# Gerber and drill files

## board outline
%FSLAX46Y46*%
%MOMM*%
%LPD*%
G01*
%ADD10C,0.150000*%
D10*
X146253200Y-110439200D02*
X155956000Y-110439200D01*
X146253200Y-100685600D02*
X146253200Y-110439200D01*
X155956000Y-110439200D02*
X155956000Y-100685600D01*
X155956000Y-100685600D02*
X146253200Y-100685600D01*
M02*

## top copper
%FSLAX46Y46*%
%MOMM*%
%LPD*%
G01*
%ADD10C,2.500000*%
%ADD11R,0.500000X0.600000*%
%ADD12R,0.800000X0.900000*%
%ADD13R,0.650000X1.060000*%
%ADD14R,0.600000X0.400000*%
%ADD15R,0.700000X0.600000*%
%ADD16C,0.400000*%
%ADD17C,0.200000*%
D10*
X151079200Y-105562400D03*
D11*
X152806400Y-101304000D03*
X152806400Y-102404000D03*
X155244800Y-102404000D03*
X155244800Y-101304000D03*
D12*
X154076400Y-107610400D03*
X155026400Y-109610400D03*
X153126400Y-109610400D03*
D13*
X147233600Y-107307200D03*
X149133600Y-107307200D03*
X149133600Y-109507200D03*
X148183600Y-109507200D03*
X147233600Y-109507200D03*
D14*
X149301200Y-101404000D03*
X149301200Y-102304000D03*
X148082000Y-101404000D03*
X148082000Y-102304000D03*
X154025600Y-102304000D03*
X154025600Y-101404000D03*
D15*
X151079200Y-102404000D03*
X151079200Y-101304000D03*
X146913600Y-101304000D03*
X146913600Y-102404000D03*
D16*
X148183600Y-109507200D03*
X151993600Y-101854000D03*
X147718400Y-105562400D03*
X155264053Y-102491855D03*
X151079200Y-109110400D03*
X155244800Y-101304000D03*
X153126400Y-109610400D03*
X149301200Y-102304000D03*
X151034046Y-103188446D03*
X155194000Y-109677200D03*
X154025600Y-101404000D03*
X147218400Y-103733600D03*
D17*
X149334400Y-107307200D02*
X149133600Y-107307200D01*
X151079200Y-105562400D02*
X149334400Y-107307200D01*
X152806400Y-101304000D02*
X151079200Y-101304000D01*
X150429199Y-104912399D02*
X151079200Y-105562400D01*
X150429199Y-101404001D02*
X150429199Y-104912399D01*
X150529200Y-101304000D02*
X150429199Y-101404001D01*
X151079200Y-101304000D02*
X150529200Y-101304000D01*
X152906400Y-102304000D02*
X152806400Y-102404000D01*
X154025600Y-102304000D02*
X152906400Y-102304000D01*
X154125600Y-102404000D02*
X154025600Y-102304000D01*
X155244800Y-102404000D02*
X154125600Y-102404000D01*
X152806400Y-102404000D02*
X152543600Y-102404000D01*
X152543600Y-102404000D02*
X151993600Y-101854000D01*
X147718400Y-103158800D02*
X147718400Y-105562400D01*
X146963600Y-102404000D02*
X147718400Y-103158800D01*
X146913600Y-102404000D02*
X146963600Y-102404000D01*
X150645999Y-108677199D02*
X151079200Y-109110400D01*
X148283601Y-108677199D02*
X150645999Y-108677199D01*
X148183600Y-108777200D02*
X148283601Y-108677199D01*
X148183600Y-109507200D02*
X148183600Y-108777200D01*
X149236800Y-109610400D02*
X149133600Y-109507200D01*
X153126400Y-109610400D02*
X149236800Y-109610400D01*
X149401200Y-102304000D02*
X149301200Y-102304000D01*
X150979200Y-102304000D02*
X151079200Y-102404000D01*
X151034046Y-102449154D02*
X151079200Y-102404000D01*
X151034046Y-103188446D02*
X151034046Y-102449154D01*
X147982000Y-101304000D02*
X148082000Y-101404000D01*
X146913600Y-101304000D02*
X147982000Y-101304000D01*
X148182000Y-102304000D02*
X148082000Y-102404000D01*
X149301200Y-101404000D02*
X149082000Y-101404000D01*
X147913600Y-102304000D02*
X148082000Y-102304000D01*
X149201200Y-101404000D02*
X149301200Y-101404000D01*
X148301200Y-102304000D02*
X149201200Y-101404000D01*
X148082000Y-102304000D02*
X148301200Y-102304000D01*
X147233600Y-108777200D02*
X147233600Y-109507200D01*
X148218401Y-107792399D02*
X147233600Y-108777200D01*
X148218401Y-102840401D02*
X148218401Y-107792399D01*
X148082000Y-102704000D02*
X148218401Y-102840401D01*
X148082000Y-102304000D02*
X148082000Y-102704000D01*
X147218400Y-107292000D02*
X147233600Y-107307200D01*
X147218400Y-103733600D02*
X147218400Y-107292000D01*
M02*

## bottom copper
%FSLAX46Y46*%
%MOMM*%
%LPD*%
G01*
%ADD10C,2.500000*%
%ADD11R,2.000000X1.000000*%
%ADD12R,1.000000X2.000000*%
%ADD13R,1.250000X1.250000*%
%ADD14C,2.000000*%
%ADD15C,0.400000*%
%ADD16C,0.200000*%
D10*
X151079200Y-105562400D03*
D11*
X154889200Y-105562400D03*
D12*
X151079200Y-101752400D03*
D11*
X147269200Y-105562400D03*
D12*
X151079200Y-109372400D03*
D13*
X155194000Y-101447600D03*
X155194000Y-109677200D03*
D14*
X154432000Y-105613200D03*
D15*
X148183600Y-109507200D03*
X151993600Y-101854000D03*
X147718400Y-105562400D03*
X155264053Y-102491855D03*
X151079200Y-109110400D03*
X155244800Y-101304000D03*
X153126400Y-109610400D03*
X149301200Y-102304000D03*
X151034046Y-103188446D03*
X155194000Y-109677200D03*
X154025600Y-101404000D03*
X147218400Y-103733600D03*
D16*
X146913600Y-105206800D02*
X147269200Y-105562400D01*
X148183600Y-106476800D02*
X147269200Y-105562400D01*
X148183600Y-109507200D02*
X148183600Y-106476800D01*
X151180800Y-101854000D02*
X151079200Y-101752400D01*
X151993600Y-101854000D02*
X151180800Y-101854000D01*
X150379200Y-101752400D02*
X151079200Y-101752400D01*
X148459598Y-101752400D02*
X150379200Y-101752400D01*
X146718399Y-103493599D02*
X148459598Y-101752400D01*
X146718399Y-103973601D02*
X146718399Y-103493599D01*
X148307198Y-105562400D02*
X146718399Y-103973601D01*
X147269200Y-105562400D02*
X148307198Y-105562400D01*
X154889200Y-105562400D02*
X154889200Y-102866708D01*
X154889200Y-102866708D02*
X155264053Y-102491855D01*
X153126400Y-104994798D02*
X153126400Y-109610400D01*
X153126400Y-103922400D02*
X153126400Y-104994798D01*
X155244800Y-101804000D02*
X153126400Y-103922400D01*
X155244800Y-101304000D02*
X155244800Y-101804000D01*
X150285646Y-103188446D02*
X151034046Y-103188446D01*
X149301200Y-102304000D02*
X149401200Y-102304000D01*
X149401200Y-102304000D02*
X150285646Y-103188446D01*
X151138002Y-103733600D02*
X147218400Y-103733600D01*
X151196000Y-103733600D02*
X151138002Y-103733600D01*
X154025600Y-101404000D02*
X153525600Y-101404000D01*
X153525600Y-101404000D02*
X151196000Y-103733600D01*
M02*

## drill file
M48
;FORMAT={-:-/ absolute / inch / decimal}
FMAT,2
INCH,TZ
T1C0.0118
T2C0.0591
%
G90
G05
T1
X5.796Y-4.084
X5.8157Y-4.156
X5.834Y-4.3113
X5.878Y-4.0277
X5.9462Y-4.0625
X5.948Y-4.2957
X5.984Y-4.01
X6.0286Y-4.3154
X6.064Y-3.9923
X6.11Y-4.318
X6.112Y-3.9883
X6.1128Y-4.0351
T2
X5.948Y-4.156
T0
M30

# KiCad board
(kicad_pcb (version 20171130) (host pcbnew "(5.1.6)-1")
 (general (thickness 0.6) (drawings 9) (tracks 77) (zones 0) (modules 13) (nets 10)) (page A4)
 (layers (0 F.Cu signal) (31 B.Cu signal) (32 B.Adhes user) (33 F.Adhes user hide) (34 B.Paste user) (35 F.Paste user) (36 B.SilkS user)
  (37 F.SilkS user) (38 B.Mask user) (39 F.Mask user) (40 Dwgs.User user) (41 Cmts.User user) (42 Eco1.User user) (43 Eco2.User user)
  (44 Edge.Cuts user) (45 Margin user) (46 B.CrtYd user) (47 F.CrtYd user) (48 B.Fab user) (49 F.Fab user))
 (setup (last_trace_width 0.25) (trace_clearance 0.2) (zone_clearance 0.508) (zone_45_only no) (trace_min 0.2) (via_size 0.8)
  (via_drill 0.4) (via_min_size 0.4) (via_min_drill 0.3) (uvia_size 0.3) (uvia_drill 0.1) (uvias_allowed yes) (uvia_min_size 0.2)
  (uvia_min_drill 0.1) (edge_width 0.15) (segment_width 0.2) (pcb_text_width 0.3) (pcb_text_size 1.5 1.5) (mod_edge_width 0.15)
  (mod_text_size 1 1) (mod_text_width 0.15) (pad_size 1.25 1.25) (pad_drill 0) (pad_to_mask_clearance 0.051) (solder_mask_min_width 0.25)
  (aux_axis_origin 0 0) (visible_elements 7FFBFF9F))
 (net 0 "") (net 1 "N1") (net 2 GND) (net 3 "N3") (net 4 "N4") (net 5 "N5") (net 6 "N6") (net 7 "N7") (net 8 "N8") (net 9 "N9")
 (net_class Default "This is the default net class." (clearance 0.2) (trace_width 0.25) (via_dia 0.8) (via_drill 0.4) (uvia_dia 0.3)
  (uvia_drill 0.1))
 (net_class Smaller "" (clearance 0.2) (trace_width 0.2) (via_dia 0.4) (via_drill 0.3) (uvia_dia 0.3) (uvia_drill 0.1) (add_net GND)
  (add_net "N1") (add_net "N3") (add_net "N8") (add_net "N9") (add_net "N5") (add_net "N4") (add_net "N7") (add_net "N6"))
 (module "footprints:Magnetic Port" (layer B.Cu) (at 151.0792 105.5624)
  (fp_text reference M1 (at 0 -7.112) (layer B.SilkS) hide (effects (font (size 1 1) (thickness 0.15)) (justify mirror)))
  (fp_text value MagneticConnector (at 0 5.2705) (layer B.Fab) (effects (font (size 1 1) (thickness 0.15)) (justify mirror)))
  (pad 1 thru_hole circle (at 0 0) (size 2.5 2.5) (drill 1.5) (layers *.Cu *.Mask) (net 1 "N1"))
  (pad 2 smd rect (at 3.81 0) (size 2 1) (layers B.Cu B.Paste B.Mask) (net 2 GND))
  (pad 2 smd rect (at 0 -3.81 270) (size 2 1) (layers B.Cu B.Paste B.Mask) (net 2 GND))
  (pad 2 smd rect (at -3.81 0) (size 2 1) (layers B.Cu B.Paste B.Mask) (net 2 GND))
  (pad 2 smd rect (at 0 3.81 270) (size 2 1) (layers B.Cu B.Paste B.Mask) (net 2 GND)))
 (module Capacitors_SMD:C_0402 (layer F.Cu) (at 152.8064 101.854 270)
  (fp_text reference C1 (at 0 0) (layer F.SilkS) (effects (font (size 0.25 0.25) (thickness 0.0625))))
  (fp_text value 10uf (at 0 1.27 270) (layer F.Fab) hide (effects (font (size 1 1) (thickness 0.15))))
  (pad 1 smd rect (at -0.55 0 270) (size 0.6 0.5) (layers F.Cu F.Paste F.Mask) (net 1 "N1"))
  (pad 2 smd rect (at 0.55 0 270) (size 0.6 0.5) (layers F.Cu F.Paste F.Mask) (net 2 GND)))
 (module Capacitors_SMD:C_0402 (layer F.Cu) (at 155.2448 101.854 270)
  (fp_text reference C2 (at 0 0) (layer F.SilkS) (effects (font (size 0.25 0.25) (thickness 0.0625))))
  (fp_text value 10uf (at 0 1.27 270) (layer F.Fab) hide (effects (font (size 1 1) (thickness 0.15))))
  (pad 2 smd rect (at 0.55 0 270) (size 0.6 0.5) (layers F.Cu F.Paste F.Mask) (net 2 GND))
  (pad 1 smd rect (at -0.55 0 270) (size 0.6 0.5) (layers F.Cu F.Paste F.Mask) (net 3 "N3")))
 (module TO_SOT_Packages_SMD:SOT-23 (layer F.Cu) (at 154.0764 108.6104 90)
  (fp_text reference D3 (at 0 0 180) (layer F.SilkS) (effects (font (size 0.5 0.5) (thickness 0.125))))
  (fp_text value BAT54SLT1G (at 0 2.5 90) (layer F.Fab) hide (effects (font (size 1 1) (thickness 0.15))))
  (pad 3 smd rect (at 1 0 90) (size 0.9 0.8) (layers F.Cu F.Paste F.Mask) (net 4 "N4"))
  (pad 2 smd rect (at -1 0.95 90) (size 0.9 0.8) (layers F.Cu F.Paste F.Mask) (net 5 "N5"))
  (pad 1 smd rect (at -1 -0.95 90) (size 0.9 0.8) (layers F.Cu F.Paste F.Mask) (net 3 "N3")))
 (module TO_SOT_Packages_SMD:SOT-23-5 (layer F.Cu) (at 148.1836 108.4072 90)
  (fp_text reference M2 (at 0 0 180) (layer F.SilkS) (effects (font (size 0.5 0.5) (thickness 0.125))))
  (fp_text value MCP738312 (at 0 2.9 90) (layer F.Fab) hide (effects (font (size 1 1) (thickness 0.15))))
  (pad 5 smd rect (at 1.1 -0.95 90) (size 1.06 0.65) (layers F.Cu F.Paste F.Mask) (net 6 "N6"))
  (pad 4 smd rect (at 1.1 0.95 90) (size 1.06 0.65) (layers F.Cu F.Paste F.Mask) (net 1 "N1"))
  (pad 3 smd rect (at -1.1 0.95 90) (size 1.06 0.65) (layers F.Cu F.Paste F.Mask) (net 3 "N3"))
  (pad 2 smd rect (at -1.1 0 90) (size 1.06 0.65) (layers F.Cu F.Paste F.Mask) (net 2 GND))
  (pad 1 smd rect (at -1.1 -0.95 90) (size 1.06 0.65) (layers F.Cu F.Paste F.Mask) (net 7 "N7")))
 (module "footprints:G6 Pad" (layer B.Cu) (at 155.194 101.4476 90)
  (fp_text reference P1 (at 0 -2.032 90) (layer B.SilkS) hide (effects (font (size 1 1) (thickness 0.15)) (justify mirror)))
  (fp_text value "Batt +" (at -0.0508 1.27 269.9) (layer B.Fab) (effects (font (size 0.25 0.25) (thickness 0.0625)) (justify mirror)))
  (pad 1 smd rect (at 0 0 90) (size 1.25 1.25) (layers B.Cu B.Paste B.Mask) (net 3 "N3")))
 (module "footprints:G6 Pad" (layer B.Cu) (at 155.194 109.6772 90)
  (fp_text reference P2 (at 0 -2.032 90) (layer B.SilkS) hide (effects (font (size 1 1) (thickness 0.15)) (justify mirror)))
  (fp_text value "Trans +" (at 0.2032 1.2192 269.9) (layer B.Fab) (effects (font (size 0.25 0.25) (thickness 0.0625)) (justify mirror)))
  (pad 1 smd rect (at 0 0 90) (size 1.25 1.25) (layers B.Cu B.Paste B.Mask) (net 5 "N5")))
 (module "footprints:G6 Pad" (layer B.Cu) (at 154.432 105.6132 90)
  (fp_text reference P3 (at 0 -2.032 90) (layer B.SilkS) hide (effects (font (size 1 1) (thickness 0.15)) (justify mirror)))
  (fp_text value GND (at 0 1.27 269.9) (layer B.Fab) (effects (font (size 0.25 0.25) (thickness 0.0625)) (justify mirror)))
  (pad 1 smd circle (at 0 0 90) (size 2 2) (layers B.Cu B.Paste B.Mask) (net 2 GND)))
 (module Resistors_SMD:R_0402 (layer F.Cu) (at 149.3012 101.854 270)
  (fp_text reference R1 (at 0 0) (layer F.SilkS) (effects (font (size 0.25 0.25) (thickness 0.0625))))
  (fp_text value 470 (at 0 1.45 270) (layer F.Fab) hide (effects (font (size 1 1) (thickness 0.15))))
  (pad 1 smd rect (at -0.45 0 270) (size 0.4 0.6) (layers F.Cu F.Paste F.Mask) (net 7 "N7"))
  (pad 2 smd rect (at 0.45 0 270) (size 0.4 0.6) (layers F.Cu F.Paste F.Mask) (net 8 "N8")))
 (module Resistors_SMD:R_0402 (layer F.Cu) (at 148.082 101.854 90)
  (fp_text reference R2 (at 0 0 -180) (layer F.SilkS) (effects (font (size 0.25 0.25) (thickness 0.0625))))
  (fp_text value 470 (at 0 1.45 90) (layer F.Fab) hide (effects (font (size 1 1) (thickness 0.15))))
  (pad 2 smd rect (at 0.45 0 90) (size 0.4 0.6) (layers F.Cu F.Paste F.Mask) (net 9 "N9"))
  (pad 1 smd rect (at -0.45 0 90) (size 0.4 0.6) (layers F.Cu F.Paste F.Mask) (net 7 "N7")))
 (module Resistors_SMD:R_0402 (layer F.Cu) (at 154.0256 101.854 270)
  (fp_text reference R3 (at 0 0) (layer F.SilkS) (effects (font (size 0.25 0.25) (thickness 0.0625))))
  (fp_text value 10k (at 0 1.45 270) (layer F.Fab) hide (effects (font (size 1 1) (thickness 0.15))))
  (pad 2 smd rect (at 0.45 0 270) (size 0.4 0.6) (layers F.Cu F.Paste F.Mask) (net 2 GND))
  (pad 1 smd rect (at -0.45 0 270) (size 0.4 0.6) (layers F.Cu F.Paste F.Mask) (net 6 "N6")))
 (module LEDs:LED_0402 (layer F.Cu) (at 151.0792 101.854 90)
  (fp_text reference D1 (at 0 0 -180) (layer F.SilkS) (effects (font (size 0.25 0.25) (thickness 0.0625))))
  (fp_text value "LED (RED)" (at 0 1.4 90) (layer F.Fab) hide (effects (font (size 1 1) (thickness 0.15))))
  (pad 1 smd rect (at -0.55 0 270) (size 0.6 0.7) (layers F.Cu F.Paste F.Mask) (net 8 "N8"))
  (pad 2 smd rect (at 0.55 0 270) (size 0.6 0.7) (layers F.Cu F.Paste F.Mask) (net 1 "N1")))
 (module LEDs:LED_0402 (layer F.Cu) (at 146.9136 101.854 90)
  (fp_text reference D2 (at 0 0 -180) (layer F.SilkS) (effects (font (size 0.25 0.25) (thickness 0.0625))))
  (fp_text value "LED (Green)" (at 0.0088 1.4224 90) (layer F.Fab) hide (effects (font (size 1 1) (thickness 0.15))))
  (pad 2 smd rect (at 0.55 0 270) (size 0.6 0.7) (layers F.Cu F.Paste F.Mask) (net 9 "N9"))
  (pad 1 smd rect (at -0.55 0 270) (size 0.6 0.7) (layers F.Cu F.Paste F.Mask) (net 2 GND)))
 (gr_line (start 146.2532 110.4392) (end 155.956 110.4392) (layer Edge.Cuts) (width 0.15))
 (gr_line (start 146.2532 100.6856) (end 146.2532 110.4392) (layer Edge.Cuts) (width 0.15))
 (gr_line (start 155.956 110.4392) (end 155.956 100.6856) (layer Edge.Cuts) (width 0.15))
 (gr_line (start 155.956 100.6856) (end 146.2532 100.6856) (layer Edge.Cuts) (width 0.15))
 (segment (start 149.3344 107.3072) (end 149.1336 107.3072) (width 0.2) (layer F.Cu) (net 1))
 (segment (start 151.0792 105.5624) (end 149.3344 107.3072) (width 0.2) (layer F.Cu) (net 1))
 (segment (start 152.8064 101.304) (end 151.0792 101.304) (width 0.2) (layer F.Cu) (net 1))
 (segment (start 150.429199 104.912399) (end 151.0792 105.5624) (width 0.2) (layer F.Cu) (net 1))
 (segment (start 150.429199 101.404001) (end 150.429199 104.912399) (width 0.2) (layer F.Cu) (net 1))
 (segment (start 150.5292 101.304) (end 150.429199 101.404001) (width 0.2) (layer F.Cu) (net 1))
 (segment (start 151.0792 101.304) (end 150.5292 101.304) (width 0.2) (layer F.Cu) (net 1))
 (segment (start 146.9136 105.2068) (end 147.2692 105.5624) (width 0.2) (layer B.Cu) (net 2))
 (via (at 148.1836 109.5072) (size 0.4) (drill 0.3) (layers F.Cu B.Cu) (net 2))
 (segment (start 148.1836 106.4768) (end 147.2692 105.5624) (width 0.2) (layer B.Cu) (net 2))
 (segment (start 148.1836 109.5072) (end 148.1836 106.4768) (width 0.2) (layer B.Cu) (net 2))
 (segment (start 152.9064 102.304) (end 152.8064 102.404) (width 0.2) (layer F.Cu) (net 2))
 (segment (start 154.0256 102.304) (end 152.9064 102.304) (width 0.2) (layer F.Cu) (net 2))
 (segment (start 154.1256 102.404) (end 154.0256 102.304) (width 0.2) (layer F.Cu) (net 2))
 (segment (start 155.2448 102.404) (end 154.1256 102.404) (width 0.2) (layer F.Cu) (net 2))
 (via (at 151.9936 101.854) (size 0.4) (drill 0.3) (layers F.Cu B.Cu) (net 2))
 (segment (start 152.8064 102.404) (end 152.5436 102.404) (width 0.2) (layer F.Cu) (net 2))
 (segment (start 152.5436 102.404) (end 151.9936 101.854) (width 0.2) (layer F.Cu) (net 2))
 (segment (start 151.1808 101.854) (end 151.0792 101.7524) (width 0.2) (layer B.Cu) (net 2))
 (segment (start 151.9936 101.854) (end 151.1808 101.854) (width 0.2) (layer B.Cu) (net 2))
 (via (at 147.7184 105.5624) (size 0.4) (drill 0.3) (layers F.Cu B.Cu) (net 2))
 (segment (start 147.7184 103.1588) (end 147.7184 105.5624) (width 0.2) (layer F.Cu) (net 2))
 (segment (start 146.9636 102.404) (end 147.7184 103.1588) (width 0.2) (layer F.Cu) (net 2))
 (segment (start 146.9136 102.404) (end 146.9636 102.404) (width 0.2) (layer F.Cu) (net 2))
 (segment (start 150.3792 101.7524) (end 151.0792 101.7524) (width 0.2) (layer B.Cu) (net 2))
 (segment (start 148.459598 101.7524) (end 150.3792 101.7524) (width 0.2) (layer B.Cu) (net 2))
 (segment (start 146.718399 103.493599) (end 148.459598 101.7524) (width 0.2) (layer B.Cu) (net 2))
 (segment (start 146.718399 103.973601) (end 146.718399 103.493599) (width 0.2) (layer B.Cu) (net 2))
 (segment (start 148.307198 105.5624) (end 146.718399 103.973601) (width 0.2) (layer B.Cu) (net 2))
 (segment (start 147.2692 105.5624) (end 148.307198 105.5624) (width 0.2) (layer B.Cu) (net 2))
 (via (at 155.264053 102.491855) (size 0.4) (drill 0.3) (layers F.Cu B.Cu) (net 2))
 (segment (start 154.8892 105.5624) (end 154.8892 102.866708) (width 0.2) (layer B.Cu) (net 2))
 (segment (start 154.8892 102.866708) (end 155.264053 102.491855) (width 0.2) (layer B.Cu) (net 2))
 (via (at 151.0792 109.1104) (size 0.4) (drill 0.3) (layers F.Cu B.Cu) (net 2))
 (segment (start 150.645999 108.677199) (end 151.0792 109.1104) (width 0.2) (layer F.Cu) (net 2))
 (segment (start 148.283601 108.677199) (end 150.645999 108.677199) (width 0.2) (layer F.Cu) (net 2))
 (segment (start 148.1836 108.7772) (end 148.283601 108.677199) (width 0.2) (layer F.Cu) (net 2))
 (segment (start 148.1836 109.5072) (end 148.1836 108.7772) (width 0.2) (layer F.Cu) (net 2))
 (via (at 155.2448 101.304) (size 0.4) (drill 0.3) (layers F.Cu B.Cu) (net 3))
 (via (at 153.1264 109.6104) (size 0.4) (drill 0.3) (layers F.Cu B.Cu) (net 3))
 (segment (start 153.1264 104.994798) (end 153.1264 109.6104) (width 0.2) (layer B.Cu) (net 3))
 (segment (start 153.1264 103.9224) (end 153.1264 104.994798) (width 0.2) (layer B.Cu) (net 3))
 (segment (start 155.2448 101.804) (end 153.1264 103.9224) (width 0.2) (layer B.Cu) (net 3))
 (segment (start 155.2448 101.304) (end 155.2448 101.804) (width 0.2) (layer B.Cu) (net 3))
 (segment (start 149.2368 109.6104) (end 149.1336 109.5072) (width 0.2) (layer F.Cu) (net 3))
 (segment (start 153.1264 109.6104) (end 149.2368 109.6104) (width 0.2) (layer F.Cu) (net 3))
 (segment (start 149.4012 102.304) (end 149.3012 102.304) (width 0.2) (layer F.Cu) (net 8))
 (segment (start 150.9792 102.304) (end 151.0792 102.404) (width 0.2) (layer F.Cu) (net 8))
 (via (at 149.3012 102.304) (size 0.4) (drill 0.3) (layers F.Cu B.Cu) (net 8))
 (via (at 151.034046 103.188446) (size 0.4) (drill 0.3) (layers F.Cu B.Cu) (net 8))
 (segment (start 150.285646 103.188446) (end 151.034046 103.188446) (width 0.2) (layer B.Cu) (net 8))
 (segment (start 149.3012 102.304) (end 149.4012 102.304) (width 0.2) (layer B.Cu) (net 8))
 (segment (start 149.4012 102.304) (end 150.285646 103.188446) (width 0.2) (layer B.Cu) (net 8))
 (segment (start 151.034046 102.449154) (end 151.0792 102.404) (width 0.2) (layer F.Cu) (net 8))
 (segment (start 151.034046 103.188446) (end 151.034046 102.449154) (width 0.2) (layer F.Cu) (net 8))
 (segment (start 147.982 101.304) (end 148.082 101.404) (width 0.2) (layer F.Cu) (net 9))
 (segment (start 146.9136 101.304) (end 147.982 101.304) (width 0.2) (layer F.Cu) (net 9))
 (via (at 155.194 109.6772) (size 0.4) (drill 0.3) (layers F.Cu B.Cu) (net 5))
 (segment (start 148.182 102.304) (end 148.082 102.404) (width 0.2) (layer F.Cu) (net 7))
 (segment (start 149.3012 101.404) (end 149.082 101.404) (width 0.2) (layer F.Cu) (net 7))
 (segment (start 147.9136 102.304) (end 148.082 102.304) (width 0.2) (layer F.Cu) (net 7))
 (segment (start 149.2012 101.404) (end 149.3012 101.404) (width 0.2) (layer F.Cu) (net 7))
 (segment (start 148.3012 102.304) (end 149.2012 101.404) (width 0.2) (layer F.Cu) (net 7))
 (segment (start 148.082 102.304) (end 148.3012 102.304) (width 0.2) (layer F.Cu) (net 7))
 (segment (start 147.2336 108.7772) (end 147.2336 109.5072) (width 0.2) (layer F.Cu) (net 7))
 (segment (start 148.218401 107.792399) (end 147.2336 108.7772) (width 0.2) (layer F.Cu) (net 7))
 (segment (start 148.218401 102.840401) (end 148.218401 107.792399) (width 0.2) (layer F.Cu) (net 7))
 (segment (start 148.082 102.704) (end 148.218401 102.840401) (width 0.2) (layer F.Cu) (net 7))
 (segment (start 148.082 102.304) (end 148.082 102.704) (width 0.2) (layer F.Cu) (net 7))
 (via (at 154.0256 101.404) (size 0.4) (drill 0.3) (layers F.Cu B.Cu) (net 6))
 (via (at 147.2184 103.7336) (size 0.4) (drill 0.3) (layers F.Cu B.Cu) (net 6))
 (segment (start 151.138002 103.7336) (end 147.2184 103.7336) (width 0.2) (layer B.Cu) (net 6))
 (segment (start 151.196 103.7336) (end 151.138002 103.7336) (width 0.2) (layer B.Cu) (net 6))
 (segment (start 154.0256 101.404) (end 153.5256 101.404) (width 0.2) (layer B.Cu) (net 6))
 (segment (start 153.5256 101.404) (end 151.196 103.7336) (width 0.2) (layer B.Cu) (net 6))
 (segment (start 147.2184 107.292) (end 147.2336 107.3072) (width 0.2) (layer F.Cu) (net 6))
 (segment (start 147.2184 103.7336) (end 147.2184 107.292) (width 0.2) (layer F.Cu) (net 6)))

